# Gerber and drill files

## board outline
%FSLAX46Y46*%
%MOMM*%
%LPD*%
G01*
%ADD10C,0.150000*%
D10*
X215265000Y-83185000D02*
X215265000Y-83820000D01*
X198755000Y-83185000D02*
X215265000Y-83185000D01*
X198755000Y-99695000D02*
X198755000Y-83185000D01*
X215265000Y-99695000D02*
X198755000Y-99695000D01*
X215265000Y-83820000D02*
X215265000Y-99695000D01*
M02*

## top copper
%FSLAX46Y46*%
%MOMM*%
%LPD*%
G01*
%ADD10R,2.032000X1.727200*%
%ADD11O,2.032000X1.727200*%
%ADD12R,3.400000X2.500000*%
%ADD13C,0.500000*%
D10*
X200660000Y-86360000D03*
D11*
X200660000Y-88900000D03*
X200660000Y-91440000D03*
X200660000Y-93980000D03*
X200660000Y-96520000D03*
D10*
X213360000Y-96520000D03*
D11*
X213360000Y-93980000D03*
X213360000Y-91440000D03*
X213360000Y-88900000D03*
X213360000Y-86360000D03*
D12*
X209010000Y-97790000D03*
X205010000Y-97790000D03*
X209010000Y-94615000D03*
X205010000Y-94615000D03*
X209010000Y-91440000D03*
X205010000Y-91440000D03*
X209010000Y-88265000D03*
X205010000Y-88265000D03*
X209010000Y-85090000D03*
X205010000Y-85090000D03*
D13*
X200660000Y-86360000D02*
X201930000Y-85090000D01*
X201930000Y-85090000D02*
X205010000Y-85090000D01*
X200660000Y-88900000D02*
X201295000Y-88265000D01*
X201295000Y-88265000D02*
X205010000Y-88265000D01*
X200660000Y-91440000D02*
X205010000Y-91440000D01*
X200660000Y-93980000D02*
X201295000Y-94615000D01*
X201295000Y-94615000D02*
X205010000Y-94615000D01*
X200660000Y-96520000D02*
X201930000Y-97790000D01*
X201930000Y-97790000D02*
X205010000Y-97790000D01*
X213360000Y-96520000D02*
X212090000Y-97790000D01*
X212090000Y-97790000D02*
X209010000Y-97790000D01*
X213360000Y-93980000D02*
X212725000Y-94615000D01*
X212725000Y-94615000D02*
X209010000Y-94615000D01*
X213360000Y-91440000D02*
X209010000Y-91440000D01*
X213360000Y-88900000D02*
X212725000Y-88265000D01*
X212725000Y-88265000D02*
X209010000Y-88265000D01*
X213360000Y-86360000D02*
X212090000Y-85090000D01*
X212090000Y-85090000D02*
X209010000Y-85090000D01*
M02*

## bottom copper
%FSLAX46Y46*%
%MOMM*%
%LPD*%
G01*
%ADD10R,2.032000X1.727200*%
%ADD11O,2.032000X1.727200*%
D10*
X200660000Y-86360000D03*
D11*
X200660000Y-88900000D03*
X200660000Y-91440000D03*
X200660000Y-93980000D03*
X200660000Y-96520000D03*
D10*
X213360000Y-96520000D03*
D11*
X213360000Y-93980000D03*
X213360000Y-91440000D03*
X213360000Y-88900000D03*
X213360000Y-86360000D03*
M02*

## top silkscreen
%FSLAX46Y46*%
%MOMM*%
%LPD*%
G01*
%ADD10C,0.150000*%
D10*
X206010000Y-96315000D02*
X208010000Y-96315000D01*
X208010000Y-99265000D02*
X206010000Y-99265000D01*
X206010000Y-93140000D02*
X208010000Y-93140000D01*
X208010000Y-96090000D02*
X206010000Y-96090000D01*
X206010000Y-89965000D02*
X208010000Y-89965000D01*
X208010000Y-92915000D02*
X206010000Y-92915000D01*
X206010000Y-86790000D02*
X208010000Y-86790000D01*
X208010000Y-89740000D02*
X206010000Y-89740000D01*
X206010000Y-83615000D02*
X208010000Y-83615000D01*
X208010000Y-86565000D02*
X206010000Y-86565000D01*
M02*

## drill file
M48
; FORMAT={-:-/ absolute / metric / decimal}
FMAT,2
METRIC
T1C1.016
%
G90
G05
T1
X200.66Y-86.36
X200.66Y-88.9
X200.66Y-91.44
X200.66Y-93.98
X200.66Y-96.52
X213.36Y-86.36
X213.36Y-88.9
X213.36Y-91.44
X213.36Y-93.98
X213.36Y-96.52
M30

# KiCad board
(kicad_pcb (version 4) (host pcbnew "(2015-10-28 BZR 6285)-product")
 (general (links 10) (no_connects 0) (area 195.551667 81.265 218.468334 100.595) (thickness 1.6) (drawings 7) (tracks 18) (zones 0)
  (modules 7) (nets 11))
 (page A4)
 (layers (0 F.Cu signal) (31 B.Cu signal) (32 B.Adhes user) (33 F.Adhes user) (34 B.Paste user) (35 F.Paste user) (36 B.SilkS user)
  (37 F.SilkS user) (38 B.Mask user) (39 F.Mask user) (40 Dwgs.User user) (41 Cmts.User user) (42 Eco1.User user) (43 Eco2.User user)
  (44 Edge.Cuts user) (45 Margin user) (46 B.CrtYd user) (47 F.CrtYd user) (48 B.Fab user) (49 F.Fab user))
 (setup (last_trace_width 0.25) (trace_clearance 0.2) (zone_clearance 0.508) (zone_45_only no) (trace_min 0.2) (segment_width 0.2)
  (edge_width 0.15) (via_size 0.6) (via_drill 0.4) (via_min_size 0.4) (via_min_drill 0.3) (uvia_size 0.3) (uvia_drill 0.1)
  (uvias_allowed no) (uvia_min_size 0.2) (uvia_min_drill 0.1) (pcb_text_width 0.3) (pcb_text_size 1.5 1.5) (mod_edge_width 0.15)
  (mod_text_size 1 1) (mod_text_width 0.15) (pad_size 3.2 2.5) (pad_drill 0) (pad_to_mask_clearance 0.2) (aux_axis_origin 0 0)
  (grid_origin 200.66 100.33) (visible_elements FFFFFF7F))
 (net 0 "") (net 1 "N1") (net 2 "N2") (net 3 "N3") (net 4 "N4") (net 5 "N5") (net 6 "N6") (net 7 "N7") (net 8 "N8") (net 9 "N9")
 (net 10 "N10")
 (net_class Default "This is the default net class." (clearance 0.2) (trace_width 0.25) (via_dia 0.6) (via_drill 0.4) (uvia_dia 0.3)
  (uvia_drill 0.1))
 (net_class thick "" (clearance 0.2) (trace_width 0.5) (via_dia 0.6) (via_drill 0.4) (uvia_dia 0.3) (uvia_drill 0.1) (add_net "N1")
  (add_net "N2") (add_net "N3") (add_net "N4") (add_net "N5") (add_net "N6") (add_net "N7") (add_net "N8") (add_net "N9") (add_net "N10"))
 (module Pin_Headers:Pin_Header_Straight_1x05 (layer B.Cu) (at 200.66 86.36 180)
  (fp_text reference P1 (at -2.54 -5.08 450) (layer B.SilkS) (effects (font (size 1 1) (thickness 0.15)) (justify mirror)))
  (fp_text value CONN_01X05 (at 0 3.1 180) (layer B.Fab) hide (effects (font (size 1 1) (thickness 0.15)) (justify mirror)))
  (pad 1 thru_hole rect (at 0 0 180) (size 2.032 1.7272) (drill 1.016) (layers *.Cu *.Mask B.SilkS) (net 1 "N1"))
  (pad 2 thru_hole oval (at 0 -2.54 180) (size 2.032 1.7272) (drill 1.016) (layers *.Cu *.Mask B.SilkS) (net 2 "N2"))
  (pad 3 thru_hole oval (at 0 -5.08 180) (size 2.032 1.7272) (drill 1.016) (layers *.Cu *.Mask B.SilkS) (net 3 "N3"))
  (pad 4 thru_hole oval (at 0 -7.62 180) (size 2.032 1.7272) (drill 1.016) (layers *.Cu *.Mask B.SilkS) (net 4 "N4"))
  (pad 5 thru_hole oval (at 0 -10.16 180) (size 2.032 1.7272) (drill 1.016) (layers *.Cu *.Mask B.SilkS) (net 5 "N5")))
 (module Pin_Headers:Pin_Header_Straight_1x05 (layer B.Cu) (at 213.36 96.52)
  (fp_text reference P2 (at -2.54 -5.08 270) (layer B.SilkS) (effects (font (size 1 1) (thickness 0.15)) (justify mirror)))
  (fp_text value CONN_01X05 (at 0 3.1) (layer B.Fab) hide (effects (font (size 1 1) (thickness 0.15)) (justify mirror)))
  (pad 1 thru_hole rect (at 0 0) (size 2.032 1.7272) (drill 1.016) (layers *.Cu *.Mask B.SilkS) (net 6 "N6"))
  (pad 2 thru_hole oval (at 0 -2.54) (size 2.032 1.7272) (drill 1.016) (layers *.Cu *.Mask B.SilkS) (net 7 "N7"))
  (pad 3 thru_hole oval (at 0 -5.08) (size 2.032 1.7272) (drill 1.016) (layers *.Cu *.Mask B.SilkS) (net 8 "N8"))
  (pad 4 thru_hole oval (at 0 -7.62) (size 2.032 1.7272) (drill 1.016) (layers *.Cu *.Mask B.SilkS) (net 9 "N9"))
  (pad 5 thru_hole oval (at 0 -10.16) (size 2.032 1.7272) (drill 1.016) (layers *.Cu *.Mask B.SilkS) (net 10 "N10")))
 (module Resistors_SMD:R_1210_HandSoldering (layer F.Cu) (at 207.01 97.79 180)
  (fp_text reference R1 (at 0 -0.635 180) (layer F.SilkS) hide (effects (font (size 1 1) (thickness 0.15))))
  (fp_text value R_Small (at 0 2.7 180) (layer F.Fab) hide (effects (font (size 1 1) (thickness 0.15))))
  (fp_line (start 1 1.475) (end -1 1.475) (layer F.SilkS) (width 0.15))
  (fp_line (start -1 -1.475) (end 1 -1.475) (layer F.SilkS) (width 0.15))
  (pad 1 smd rect (at -2 0 180) (size 3.4 2.5) (layers F.Cu F.Paste F.Mask) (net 6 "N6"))
  (pad 2 smd rect (at 2 0 180) (size 3.4 2.5) (layers F.Cu F.Paste F.Mask) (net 5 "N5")))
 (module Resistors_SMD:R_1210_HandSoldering (layer F.Cu) (at 207.01 94.615 180)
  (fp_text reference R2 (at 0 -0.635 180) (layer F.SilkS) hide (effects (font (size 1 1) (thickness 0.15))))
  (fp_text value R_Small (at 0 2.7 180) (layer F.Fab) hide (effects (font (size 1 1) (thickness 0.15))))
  (fp_line (start 1 1.475) (end -1 1.475) (layer F.SilkS) (width 0.15))
  (fp_line (start -1 -1.475) (end 1 -1.475) (layer F.SilkS) (width 0.15))
  (pad 1 smd rect (at -2 0 180) (size 3.4 2.5) (layers F.Cu F.Paste F.Mask) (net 7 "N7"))
  (pad 2 smd rect (at 2 0 180) (size 3.4 2.5) (layers F.Cu F.Paste F.Mask) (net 4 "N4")))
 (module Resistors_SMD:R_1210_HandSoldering (layer F.Cu) (at 207.01 91.44 180)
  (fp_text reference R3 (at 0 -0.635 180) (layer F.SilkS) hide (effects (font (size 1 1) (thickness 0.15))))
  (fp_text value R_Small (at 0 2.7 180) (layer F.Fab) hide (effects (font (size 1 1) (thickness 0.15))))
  (fp_line (start 1 1.475) (end -1 1.475) (layer F.SilkS) (width 0.15))
  (fp_line (start -1 -1.475) (end 1 -1.475) (layer F.SilkS) (width 0.15))
  (pad 1 smd rect (at -2 0 180) (size 3.4 2.5) (layers F.Cu F.Paste F.Mask) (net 8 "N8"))
  (pad 2 smd rect (at 2 0 180) (size 3.4 2.5) (layers F.Cu F.Paste F.Mask) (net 3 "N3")))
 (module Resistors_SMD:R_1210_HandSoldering (layer F.Cu) (at 207.01 88.265 180)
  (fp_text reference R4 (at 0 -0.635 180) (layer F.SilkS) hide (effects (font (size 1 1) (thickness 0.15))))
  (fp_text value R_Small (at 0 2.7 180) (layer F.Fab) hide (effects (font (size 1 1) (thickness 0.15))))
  (fp_line (start 1 1.475) (end -1 1.475) (layer F.SilkS) (width 0.15))
  (fp_line (start -1 -1.475) (end 1 -1.475) (layer F.SilkS) (width 0.15))
  (pad 1 smd rect (at -2 0 180) (size 3.4 2.5) (layers F.Cu F.Paste F.Mask) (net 9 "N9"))
  (pad 2 smd rect (at 2 0 180) (size 3.4 2.5) (layers F.Cu F.Paste F.Mask) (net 2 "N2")))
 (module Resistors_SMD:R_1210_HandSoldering (layer F.Cu) (at 207.01 85.09 180)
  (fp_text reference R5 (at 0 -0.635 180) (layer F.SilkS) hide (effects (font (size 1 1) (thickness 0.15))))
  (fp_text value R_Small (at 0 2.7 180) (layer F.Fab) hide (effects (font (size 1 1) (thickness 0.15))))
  (fp_line (start 1 1.475) (end -1 1.475) (layer F.SilkS) (width 0.15))
  (fp_line (start -1 -1.475) (end 1 -1.475) (layer F.SilkS) (width 0.15))
  (pad 1 smd rect (at -2 0 180) (size 3.4 2.5) (layers F.Cu F.Paste F.Mask) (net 10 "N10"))
  (pad 2 smd rect (at 2 0 180) (size 3.4 2.5) (layers F.Cu F.Paste F.Mask) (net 1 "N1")))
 (gr_line (start 215.265 83.185) (end 215.265 83.82) (angle 90) (layer Edge.Cuts) (width 0.15))
 (gr_line (start 198.755 83.185) (end 215.265 83.185) (angle 90) (layer Edge.Cuts) (width 0.15))
 (gr_line (start 198.755 99.695) (end 198.755 83.185) (angle 90) (layer Edge.Cuts) (width 0.15))
 (gr_line (start 215.265 99.695) (end 198.755 99.695) (angle 90) (layer Edge.Cuts) (width 0.15))
 (gr_line (start 215.265 83.82) (end 215.265 99.695) (angle 90) (layer Edge.Cuts) (width 0.15))
 (segment (start 200.66 86.36) (end 201.93 85.09) (width 0.5) (layer F.Cu) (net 1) (status 400010))
 (segment (start 201.93 85.09) (end 205.01 85.09) (width 0.5) (layer F.Cu) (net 1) (status 800020))
 (segment (start 200.66 88.9) (end 201.295 88.265) (width 0.5) (layer F.Cu) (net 2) (status C00030))
 (segment (start 201.295 88.265) (end 205.01 88.265) (width 0.5) (layer F.Cu) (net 2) (status C00030))
 (segment (start 200.66 91.44) (end 205.01 91.44) (width 0.5) (layer F.Cu) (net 3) (status C00030))
 (segment (start 200.66 93.98) (end 201.295 94.615) (width 0.5) (layer F.Cu) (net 4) (status C00030))
 (segment (start 201.295 94.615) (end 205.01 94.615) (width 0.5) (layer F.Cu) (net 4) (status C00030))
 (segment (start 200.66 96.52) (end 201.93 97.79) (width 0.5) (layer F.Cu) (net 5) (status 400010))
 (segment (start 201.93 97.79) (end 205.01 97.79) (width 0.5) (layer F.Cu) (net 5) (status 800020))
 (segment (start 213.36 96.52) (end 212.09 97.79) (width 0.5) (layer F.Cu) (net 6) (status 400010))
 (segment (start 212.09 97.79) (end 209.01 97.79) (width 0.5) (layer F.Cu) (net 6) (status 800020))
 (segment (start 213.36 93.98) (end 212.725 94.615) (width 0.5) (layer F.Cu) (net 7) (status C00030))
 (segment (start 212.725 94.615) (end 209.01 94.615) (width 0.5) (layer F.Cu) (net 7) (status C00030))
 (segment (start 213.36 91.44) (end 209.01 91.44) (width 0.5) (layer F.Cu) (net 8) (status C00030))
 (segment (start 213.36 88.9) (end 212.725 88.265) (width 0.5) (layer F.Cu) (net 9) (status C00030))
 (segment (start 212.725 88.265) (end 209.01 88.265) (width 0.5) (layer F.Cu) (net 9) (status C00030))
 (segment (start 213.36 86.36) (end 212.09 85.09) (width 0.5) (layer F.Cu) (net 10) (status 400010))
 (segment (start 212.09 85.09) (end 209.01 85.09) (width 0.5) (layer F.Cu) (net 10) (status 800020)))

